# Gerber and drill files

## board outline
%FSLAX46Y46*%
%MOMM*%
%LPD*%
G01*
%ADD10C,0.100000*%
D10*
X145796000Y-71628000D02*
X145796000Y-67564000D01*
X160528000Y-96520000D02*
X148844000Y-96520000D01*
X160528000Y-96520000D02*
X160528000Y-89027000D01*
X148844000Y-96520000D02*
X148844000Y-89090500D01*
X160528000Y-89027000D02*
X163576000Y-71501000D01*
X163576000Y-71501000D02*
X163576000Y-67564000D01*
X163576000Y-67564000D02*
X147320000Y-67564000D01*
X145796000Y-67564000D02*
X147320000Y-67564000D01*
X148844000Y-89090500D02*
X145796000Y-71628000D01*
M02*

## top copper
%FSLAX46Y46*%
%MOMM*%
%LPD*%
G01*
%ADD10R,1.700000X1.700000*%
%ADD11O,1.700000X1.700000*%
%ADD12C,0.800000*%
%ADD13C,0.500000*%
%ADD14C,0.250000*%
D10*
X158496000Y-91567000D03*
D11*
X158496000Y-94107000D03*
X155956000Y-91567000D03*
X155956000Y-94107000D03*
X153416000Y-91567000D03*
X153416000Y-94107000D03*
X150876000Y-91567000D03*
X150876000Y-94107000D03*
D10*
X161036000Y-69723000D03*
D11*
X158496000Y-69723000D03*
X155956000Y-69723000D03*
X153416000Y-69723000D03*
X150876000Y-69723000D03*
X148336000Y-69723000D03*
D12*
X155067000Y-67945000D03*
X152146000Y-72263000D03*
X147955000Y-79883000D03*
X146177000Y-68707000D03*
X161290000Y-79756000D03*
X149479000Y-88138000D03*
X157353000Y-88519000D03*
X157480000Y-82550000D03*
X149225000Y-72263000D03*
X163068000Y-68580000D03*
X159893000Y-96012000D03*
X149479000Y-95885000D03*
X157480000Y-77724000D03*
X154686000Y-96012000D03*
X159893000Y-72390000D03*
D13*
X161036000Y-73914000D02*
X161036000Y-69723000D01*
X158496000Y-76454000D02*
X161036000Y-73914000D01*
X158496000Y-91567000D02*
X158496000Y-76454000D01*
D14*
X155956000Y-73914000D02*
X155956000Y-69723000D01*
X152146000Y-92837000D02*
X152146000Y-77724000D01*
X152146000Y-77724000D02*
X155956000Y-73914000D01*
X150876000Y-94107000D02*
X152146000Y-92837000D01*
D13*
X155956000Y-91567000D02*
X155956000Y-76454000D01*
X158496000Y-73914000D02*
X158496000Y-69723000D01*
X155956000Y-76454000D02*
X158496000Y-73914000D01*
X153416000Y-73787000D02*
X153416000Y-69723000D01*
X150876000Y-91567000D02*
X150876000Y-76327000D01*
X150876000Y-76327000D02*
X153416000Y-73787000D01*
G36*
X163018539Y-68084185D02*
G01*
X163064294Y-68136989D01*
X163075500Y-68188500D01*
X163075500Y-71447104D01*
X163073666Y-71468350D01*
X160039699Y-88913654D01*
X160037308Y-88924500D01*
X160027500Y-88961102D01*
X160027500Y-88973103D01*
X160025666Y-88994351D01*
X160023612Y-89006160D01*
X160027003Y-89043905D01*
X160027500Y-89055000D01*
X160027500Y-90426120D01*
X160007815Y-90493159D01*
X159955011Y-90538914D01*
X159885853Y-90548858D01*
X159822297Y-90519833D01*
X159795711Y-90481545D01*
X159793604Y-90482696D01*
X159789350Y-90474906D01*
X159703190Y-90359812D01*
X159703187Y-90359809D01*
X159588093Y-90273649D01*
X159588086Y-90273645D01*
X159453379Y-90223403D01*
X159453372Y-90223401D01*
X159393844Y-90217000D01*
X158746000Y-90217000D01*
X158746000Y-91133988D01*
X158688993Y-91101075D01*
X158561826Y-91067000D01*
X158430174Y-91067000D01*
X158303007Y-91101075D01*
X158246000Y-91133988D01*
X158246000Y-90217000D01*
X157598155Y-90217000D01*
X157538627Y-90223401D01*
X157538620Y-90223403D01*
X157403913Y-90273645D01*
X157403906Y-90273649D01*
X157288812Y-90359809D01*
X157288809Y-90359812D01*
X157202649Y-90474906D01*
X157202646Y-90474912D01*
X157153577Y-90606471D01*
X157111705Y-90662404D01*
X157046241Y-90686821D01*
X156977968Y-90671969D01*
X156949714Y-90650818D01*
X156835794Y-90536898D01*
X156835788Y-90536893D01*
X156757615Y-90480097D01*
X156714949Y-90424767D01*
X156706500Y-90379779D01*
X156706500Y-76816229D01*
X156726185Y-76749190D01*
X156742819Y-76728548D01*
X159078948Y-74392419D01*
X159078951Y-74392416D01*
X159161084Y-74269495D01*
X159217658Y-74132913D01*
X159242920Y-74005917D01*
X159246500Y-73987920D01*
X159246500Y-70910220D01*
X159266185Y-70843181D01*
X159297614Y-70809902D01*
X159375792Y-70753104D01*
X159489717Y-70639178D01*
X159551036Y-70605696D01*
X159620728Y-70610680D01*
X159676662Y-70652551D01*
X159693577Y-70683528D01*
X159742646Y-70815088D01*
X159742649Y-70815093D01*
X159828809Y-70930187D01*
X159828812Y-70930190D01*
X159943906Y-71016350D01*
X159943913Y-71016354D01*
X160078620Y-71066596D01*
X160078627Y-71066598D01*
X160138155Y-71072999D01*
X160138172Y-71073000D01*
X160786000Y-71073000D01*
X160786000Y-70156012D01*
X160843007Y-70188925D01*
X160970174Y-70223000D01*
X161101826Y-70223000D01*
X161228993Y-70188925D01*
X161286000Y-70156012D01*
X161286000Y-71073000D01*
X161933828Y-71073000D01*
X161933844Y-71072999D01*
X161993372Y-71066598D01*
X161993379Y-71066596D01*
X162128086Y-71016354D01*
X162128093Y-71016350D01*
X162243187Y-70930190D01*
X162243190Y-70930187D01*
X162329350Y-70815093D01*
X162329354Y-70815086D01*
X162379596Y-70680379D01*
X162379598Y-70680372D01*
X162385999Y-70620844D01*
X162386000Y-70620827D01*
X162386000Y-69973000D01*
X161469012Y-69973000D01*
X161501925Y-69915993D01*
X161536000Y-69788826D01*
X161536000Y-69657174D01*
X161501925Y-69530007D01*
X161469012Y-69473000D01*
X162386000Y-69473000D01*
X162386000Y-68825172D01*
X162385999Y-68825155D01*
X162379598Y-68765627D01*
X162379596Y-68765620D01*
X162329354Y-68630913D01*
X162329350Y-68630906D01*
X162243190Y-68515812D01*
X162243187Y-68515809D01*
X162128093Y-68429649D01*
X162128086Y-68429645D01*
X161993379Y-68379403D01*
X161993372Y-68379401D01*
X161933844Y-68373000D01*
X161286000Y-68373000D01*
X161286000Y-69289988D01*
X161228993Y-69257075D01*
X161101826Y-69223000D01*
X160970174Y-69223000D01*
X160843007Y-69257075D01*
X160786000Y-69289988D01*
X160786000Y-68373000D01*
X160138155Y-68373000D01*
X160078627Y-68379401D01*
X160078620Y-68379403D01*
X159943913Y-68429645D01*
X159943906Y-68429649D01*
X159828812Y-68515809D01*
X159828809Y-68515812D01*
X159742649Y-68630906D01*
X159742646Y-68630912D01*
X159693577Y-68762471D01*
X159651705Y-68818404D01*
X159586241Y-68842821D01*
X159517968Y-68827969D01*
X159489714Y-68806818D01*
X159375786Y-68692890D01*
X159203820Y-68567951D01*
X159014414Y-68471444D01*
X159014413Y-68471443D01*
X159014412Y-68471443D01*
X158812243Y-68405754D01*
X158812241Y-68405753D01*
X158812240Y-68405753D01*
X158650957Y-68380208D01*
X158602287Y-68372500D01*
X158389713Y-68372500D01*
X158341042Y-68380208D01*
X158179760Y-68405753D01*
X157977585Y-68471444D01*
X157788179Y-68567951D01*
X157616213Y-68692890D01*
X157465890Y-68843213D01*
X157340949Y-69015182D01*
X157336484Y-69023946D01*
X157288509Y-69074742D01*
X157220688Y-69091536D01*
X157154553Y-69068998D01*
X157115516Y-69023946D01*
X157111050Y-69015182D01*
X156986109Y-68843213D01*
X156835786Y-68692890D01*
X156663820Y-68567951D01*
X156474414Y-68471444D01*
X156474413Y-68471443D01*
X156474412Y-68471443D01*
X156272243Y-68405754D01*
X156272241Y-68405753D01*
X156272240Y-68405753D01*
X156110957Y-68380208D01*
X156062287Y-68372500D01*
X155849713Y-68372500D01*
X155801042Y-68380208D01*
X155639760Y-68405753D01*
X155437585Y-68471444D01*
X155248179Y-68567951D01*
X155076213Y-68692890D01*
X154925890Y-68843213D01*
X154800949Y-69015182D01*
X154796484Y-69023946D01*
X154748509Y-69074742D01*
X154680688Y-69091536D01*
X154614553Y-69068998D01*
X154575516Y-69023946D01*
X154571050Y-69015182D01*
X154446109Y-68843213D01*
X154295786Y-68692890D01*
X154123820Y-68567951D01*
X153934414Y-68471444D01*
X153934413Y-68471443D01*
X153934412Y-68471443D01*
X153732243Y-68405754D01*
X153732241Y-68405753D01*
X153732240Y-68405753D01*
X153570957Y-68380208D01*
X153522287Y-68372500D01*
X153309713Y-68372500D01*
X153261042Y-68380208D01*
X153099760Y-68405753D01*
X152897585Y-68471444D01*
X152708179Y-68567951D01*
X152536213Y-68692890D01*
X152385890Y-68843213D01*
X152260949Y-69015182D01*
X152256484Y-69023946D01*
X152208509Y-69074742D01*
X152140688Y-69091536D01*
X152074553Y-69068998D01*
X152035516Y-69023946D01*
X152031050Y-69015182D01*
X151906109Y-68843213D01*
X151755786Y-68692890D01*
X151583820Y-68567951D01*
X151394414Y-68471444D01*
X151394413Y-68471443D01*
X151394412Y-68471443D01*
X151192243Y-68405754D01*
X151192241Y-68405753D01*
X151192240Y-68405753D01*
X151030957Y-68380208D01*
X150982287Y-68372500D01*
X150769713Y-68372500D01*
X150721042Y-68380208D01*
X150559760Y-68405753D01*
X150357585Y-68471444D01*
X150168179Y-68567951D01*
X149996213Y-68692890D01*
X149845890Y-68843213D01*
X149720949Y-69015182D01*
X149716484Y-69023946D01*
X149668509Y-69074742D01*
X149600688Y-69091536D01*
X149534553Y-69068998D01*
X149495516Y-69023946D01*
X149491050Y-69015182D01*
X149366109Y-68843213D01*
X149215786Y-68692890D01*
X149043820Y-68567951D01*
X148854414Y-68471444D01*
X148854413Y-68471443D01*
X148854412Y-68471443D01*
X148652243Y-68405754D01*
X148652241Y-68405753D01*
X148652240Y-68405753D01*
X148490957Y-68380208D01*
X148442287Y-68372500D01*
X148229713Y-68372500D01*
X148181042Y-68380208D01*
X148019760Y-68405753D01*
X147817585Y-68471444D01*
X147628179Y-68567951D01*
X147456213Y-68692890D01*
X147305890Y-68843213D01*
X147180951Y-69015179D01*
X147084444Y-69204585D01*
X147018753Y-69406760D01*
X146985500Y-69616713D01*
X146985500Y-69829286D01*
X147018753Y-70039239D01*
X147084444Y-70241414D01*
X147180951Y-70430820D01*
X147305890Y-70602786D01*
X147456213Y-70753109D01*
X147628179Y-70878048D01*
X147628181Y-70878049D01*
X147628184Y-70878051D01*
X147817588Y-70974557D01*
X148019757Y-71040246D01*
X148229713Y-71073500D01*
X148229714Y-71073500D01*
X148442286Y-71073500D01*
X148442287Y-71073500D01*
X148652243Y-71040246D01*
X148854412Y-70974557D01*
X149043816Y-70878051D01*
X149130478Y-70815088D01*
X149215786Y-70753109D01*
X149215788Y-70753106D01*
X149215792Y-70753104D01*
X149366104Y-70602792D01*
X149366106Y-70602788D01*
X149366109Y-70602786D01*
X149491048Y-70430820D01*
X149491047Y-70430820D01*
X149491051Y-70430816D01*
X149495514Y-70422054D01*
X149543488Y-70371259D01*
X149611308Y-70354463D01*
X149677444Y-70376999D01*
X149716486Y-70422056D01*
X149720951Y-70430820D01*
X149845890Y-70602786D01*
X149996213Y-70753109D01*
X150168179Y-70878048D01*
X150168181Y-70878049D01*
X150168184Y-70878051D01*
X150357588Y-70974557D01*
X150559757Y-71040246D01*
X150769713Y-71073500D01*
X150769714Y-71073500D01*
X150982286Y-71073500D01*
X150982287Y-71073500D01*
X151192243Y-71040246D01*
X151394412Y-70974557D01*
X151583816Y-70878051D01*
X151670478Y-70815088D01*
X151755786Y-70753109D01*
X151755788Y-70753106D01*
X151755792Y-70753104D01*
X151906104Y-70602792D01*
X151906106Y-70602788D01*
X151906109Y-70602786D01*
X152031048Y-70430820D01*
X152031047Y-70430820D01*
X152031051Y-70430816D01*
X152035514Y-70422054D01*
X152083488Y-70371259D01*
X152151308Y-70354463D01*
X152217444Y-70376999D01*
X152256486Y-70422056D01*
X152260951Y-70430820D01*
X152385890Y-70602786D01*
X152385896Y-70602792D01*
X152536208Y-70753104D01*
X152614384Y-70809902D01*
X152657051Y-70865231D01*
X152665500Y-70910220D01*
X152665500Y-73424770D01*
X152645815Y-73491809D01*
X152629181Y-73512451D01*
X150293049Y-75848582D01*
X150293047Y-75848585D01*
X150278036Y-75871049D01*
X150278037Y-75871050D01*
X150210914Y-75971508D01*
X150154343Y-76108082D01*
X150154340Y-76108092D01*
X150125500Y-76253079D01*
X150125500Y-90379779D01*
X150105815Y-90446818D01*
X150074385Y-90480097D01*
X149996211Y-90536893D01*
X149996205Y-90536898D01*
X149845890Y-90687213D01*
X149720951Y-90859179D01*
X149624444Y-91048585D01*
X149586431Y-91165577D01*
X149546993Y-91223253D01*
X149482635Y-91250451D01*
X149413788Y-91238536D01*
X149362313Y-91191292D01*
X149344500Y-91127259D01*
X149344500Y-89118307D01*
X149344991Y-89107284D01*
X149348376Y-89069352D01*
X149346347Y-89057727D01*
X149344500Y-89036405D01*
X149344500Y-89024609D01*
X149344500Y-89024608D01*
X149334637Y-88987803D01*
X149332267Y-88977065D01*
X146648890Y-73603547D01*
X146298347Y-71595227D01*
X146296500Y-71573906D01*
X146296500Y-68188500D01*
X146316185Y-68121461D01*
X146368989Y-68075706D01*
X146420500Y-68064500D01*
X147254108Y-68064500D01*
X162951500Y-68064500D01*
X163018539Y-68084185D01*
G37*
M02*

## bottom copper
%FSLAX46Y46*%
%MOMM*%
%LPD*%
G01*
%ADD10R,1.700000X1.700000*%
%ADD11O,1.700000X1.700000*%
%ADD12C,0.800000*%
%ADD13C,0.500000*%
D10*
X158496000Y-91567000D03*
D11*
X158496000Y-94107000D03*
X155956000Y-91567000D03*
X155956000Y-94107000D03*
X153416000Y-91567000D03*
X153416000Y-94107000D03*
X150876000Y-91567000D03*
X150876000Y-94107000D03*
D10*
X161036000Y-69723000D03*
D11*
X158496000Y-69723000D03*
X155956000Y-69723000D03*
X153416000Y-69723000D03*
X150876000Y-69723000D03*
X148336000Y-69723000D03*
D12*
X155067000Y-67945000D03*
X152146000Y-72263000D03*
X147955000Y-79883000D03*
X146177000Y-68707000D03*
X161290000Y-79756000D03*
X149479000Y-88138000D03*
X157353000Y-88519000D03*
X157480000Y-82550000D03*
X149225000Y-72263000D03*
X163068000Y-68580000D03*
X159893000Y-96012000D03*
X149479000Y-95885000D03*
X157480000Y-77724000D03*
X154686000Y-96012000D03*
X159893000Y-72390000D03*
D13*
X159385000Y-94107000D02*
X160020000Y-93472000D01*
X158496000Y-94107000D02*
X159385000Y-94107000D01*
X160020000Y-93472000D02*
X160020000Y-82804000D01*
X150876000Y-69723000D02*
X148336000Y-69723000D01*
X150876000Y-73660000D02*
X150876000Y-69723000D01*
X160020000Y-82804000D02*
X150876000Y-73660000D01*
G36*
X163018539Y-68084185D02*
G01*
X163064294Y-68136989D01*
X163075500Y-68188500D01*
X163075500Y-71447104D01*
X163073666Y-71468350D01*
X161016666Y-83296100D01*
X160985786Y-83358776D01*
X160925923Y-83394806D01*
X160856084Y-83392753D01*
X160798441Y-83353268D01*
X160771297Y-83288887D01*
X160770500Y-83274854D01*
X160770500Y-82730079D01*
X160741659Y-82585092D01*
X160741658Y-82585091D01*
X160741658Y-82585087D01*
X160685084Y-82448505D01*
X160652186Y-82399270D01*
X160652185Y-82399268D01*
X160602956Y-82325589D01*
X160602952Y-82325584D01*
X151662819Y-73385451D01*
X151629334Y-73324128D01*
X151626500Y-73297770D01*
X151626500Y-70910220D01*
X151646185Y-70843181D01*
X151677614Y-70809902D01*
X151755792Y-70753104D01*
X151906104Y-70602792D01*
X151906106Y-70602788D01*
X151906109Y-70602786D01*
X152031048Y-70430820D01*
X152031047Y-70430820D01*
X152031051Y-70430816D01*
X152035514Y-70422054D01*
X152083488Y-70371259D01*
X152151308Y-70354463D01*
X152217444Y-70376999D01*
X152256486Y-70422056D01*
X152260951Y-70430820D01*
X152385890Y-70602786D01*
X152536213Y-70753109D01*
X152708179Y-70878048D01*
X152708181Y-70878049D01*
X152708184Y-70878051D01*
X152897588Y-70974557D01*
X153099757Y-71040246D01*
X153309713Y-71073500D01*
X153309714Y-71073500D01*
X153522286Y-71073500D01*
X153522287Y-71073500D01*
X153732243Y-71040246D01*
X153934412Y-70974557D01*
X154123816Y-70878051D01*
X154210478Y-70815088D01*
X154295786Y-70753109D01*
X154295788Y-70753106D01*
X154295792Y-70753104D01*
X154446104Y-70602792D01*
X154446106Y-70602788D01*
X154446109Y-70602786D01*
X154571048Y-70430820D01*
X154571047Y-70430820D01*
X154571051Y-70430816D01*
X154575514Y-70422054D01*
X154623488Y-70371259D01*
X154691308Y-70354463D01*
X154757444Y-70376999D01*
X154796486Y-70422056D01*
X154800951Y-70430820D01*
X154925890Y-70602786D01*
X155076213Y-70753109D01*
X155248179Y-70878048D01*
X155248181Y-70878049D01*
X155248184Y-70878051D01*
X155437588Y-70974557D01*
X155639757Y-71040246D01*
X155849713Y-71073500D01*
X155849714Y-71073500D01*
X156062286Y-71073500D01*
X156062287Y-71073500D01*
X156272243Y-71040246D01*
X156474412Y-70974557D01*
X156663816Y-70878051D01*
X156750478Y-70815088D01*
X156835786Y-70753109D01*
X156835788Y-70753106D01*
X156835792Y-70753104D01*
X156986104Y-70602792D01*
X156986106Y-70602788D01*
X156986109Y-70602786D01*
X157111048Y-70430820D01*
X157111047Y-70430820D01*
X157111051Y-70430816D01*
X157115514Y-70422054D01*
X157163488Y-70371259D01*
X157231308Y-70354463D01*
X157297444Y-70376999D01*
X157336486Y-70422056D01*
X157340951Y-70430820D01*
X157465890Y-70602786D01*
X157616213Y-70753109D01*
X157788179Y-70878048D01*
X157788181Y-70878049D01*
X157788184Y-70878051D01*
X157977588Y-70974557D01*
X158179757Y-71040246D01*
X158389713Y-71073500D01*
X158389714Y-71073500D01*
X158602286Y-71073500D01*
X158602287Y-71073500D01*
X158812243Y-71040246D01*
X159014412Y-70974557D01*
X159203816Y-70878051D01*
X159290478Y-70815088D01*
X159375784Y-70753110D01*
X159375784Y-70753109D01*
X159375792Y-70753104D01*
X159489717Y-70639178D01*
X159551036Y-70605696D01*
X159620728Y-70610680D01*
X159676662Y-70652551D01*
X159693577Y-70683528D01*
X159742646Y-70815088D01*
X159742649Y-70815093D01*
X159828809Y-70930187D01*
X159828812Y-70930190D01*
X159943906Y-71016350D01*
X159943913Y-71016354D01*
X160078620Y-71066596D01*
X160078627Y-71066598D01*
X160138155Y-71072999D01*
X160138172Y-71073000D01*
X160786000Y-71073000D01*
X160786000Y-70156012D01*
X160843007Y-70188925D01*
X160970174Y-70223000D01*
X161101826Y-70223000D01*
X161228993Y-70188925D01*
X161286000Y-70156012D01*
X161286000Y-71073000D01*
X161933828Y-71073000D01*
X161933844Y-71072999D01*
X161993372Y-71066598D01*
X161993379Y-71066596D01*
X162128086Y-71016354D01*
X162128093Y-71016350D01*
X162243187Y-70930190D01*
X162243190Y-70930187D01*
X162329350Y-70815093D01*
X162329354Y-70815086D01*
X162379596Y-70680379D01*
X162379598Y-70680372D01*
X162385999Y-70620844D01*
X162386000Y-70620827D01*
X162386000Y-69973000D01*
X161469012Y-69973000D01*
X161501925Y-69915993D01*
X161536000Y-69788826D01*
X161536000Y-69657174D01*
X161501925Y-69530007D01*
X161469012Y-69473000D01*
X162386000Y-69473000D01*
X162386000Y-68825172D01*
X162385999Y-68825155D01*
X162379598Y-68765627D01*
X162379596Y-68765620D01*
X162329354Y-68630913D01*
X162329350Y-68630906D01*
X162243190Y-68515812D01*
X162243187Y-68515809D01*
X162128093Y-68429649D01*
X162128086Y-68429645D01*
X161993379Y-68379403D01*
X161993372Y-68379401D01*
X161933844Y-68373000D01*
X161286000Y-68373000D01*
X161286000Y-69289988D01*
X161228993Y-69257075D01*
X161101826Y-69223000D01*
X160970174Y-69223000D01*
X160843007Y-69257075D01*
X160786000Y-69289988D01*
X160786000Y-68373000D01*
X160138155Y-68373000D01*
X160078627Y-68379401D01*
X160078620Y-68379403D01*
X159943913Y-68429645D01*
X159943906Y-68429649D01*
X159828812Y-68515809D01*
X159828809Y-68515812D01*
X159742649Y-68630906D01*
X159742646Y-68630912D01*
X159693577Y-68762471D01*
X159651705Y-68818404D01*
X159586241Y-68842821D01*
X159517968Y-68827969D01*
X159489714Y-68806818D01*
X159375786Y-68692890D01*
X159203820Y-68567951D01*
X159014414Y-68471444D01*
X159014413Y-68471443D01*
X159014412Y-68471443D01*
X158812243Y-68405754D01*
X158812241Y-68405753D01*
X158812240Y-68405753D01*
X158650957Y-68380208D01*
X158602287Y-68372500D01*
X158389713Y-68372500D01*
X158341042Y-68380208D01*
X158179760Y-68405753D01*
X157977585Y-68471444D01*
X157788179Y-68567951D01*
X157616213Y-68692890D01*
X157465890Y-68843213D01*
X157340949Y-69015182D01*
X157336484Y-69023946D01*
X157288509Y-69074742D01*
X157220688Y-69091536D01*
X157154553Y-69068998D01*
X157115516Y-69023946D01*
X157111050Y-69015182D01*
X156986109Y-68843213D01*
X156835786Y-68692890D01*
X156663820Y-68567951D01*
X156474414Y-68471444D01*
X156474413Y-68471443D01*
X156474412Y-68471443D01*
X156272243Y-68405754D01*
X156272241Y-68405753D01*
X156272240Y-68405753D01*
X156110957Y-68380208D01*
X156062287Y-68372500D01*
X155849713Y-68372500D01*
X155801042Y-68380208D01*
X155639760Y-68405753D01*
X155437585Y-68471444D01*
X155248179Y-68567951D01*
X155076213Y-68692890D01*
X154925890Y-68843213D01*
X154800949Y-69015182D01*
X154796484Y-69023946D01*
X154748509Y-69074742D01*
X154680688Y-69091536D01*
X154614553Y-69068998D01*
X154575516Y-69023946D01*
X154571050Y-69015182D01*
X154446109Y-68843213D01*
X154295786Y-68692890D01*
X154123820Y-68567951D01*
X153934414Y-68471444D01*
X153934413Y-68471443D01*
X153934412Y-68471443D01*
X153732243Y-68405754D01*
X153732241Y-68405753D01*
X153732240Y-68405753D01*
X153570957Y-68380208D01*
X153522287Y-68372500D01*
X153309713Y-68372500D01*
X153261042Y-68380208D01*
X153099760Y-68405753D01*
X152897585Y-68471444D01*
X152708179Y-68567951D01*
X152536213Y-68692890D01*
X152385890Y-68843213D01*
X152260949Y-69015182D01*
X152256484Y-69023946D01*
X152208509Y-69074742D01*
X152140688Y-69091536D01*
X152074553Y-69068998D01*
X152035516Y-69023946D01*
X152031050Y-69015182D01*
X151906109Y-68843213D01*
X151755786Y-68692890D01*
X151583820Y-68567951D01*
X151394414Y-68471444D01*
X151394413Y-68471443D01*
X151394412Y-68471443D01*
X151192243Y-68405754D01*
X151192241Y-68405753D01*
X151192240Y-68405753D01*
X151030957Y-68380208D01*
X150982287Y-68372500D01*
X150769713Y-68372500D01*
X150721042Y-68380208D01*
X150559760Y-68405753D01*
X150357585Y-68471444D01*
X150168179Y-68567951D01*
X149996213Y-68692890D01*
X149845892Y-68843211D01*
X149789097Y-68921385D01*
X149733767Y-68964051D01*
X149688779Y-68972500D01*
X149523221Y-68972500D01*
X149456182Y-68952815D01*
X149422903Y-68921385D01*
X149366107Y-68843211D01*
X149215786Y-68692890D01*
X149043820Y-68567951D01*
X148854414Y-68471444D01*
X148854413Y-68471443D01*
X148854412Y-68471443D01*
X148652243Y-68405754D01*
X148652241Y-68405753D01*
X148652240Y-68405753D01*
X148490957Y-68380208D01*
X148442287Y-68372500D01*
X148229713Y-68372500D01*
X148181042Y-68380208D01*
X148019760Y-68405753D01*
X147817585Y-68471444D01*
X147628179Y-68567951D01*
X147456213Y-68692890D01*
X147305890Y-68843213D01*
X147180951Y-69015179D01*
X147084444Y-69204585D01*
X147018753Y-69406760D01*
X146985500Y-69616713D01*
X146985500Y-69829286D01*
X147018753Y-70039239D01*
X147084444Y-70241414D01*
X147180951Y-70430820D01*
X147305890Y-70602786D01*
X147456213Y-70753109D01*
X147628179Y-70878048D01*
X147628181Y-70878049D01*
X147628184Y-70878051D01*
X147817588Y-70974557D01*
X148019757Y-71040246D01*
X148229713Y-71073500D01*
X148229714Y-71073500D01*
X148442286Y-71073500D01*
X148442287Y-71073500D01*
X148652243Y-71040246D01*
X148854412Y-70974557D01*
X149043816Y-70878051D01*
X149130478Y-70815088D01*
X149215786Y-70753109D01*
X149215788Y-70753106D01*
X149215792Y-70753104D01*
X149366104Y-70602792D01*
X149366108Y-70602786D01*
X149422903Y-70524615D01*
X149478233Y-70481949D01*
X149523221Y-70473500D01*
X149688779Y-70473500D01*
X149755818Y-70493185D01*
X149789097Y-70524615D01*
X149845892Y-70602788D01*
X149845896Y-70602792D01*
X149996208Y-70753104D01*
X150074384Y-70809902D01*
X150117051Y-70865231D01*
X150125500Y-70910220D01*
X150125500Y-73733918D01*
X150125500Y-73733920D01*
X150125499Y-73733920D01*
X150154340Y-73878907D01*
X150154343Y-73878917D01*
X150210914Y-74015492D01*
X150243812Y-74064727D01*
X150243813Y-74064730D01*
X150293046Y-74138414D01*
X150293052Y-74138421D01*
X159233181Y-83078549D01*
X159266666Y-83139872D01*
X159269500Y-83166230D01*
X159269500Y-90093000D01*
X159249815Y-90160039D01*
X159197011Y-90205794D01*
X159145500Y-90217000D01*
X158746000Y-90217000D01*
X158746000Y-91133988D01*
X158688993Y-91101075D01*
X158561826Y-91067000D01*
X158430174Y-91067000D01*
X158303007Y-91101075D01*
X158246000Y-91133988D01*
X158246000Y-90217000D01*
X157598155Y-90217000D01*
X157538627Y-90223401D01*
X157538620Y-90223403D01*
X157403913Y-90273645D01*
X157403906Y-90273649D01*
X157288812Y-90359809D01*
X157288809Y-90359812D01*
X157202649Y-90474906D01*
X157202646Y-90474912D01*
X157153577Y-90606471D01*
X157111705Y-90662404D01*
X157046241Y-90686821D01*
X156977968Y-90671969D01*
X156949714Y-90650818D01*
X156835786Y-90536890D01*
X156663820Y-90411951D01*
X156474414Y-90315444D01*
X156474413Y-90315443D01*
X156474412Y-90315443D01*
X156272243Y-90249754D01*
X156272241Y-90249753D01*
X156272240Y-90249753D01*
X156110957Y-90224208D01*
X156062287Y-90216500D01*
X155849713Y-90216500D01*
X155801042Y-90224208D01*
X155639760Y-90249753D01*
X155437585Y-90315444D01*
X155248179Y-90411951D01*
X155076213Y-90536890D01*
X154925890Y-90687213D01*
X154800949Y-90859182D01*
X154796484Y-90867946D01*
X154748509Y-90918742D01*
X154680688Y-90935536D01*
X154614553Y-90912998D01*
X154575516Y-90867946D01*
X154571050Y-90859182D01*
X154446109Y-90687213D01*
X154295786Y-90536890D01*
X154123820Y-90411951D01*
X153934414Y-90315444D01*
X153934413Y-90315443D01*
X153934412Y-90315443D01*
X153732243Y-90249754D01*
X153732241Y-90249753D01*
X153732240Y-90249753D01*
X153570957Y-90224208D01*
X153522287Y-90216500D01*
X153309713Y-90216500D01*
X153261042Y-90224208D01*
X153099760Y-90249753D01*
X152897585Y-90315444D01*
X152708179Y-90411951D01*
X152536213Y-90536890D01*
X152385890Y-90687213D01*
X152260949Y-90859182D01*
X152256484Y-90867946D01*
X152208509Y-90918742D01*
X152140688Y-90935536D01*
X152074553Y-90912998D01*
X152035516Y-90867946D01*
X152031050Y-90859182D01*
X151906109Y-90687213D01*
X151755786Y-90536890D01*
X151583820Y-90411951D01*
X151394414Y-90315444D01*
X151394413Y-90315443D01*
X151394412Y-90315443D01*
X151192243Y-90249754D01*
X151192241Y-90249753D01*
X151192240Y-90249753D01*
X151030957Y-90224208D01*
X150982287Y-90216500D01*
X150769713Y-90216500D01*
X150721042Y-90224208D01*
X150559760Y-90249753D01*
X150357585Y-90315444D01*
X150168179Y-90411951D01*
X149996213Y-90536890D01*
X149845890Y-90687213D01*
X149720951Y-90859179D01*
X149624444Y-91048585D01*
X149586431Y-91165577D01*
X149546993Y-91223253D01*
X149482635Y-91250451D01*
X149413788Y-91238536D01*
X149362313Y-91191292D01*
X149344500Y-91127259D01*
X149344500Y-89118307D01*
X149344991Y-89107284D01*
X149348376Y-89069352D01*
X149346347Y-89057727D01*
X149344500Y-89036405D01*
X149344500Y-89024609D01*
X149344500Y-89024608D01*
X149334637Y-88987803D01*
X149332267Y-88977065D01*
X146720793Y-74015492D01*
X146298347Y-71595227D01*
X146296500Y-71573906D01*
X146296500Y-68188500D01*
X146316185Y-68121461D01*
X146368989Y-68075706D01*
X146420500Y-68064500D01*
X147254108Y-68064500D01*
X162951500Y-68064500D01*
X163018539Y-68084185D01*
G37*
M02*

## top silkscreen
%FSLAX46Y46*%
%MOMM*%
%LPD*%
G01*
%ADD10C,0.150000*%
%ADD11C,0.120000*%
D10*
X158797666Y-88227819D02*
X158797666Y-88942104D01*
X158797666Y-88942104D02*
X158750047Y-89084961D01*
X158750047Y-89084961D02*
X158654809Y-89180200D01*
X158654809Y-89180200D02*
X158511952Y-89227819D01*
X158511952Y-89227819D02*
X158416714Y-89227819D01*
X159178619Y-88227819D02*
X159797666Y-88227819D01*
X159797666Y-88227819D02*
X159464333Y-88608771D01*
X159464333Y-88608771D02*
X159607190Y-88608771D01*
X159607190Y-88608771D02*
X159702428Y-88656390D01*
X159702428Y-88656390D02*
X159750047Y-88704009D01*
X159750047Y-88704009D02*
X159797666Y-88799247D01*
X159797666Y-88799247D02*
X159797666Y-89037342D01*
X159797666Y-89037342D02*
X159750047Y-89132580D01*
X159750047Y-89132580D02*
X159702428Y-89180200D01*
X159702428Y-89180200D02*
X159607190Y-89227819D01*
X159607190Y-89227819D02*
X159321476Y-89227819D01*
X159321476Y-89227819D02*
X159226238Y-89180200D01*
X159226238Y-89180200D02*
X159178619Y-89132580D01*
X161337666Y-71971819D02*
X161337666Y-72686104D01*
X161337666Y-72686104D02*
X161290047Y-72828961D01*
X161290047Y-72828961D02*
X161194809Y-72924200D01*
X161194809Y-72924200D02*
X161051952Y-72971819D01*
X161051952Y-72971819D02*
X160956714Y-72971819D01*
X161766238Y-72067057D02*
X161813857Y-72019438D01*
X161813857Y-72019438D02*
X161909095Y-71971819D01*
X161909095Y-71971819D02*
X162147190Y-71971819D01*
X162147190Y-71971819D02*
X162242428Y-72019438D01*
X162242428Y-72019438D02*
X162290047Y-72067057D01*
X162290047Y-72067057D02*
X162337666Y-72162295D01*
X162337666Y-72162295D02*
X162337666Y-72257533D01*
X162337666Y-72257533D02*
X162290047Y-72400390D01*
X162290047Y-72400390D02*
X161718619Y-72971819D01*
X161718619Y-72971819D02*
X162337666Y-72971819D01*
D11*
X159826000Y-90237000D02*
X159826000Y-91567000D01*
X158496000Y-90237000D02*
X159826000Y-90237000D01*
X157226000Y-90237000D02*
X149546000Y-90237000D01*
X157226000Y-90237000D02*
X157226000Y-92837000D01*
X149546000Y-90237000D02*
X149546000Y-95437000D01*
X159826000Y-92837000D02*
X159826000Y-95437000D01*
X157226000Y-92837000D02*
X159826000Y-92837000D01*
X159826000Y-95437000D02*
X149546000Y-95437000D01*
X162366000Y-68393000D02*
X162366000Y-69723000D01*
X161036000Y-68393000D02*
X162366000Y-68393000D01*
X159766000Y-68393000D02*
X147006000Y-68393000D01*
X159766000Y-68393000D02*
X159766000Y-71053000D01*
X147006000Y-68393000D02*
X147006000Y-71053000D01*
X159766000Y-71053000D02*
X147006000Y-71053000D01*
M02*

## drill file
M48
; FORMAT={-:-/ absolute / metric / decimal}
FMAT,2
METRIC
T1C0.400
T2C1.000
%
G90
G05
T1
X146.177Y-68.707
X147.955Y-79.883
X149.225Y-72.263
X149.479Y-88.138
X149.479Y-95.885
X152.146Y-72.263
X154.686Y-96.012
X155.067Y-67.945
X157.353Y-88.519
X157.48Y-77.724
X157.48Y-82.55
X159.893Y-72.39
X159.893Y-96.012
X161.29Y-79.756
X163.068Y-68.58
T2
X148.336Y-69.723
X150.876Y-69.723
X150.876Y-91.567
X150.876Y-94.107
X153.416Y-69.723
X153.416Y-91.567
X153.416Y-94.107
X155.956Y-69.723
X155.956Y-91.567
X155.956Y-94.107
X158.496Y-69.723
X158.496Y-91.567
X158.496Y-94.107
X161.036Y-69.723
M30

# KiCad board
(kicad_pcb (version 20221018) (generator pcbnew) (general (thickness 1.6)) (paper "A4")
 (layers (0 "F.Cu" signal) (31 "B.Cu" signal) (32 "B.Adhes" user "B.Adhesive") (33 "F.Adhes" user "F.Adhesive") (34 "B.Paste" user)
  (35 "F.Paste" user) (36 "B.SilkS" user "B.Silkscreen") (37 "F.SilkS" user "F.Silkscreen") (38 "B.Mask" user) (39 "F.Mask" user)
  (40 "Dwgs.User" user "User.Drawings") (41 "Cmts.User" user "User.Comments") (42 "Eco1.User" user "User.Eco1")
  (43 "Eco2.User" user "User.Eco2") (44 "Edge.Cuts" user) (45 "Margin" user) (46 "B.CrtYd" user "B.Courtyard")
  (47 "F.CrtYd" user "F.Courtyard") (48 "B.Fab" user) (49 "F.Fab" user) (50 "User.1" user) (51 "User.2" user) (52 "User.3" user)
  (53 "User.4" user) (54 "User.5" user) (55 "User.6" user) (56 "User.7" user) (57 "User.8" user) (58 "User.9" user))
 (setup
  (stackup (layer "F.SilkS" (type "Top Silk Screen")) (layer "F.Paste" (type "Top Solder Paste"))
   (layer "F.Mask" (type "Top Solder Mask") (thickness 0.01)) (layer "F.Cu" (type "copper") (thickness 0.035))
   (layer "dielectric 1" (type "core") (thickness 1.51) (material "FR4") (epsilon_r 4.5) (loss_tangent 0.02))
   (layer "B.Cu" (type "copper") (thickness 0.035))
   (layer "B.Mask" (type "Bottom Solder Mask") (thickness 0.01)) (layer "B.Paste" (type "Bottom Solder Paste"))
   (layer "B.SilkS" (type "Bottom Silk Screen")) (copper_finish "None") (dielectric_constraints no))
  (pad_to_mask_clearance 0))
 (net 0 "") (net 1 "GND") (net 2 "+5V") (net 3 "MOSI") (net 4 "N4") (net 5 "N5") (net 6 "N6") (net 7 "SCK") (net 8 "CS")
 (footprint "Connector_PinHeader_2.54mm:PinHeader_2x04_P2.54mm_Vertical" (layer "F.Cu") (at 158.496 91.567 -90)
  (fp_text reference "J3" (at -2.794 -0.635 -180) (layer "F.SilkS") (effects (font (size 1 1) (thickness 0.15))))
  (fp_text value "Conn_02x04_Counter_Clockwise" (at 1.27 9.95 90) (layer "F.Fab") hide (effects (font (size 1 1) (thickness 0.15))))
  (fp_line (start -1.33 -1.33) (end 0 -1.33) (stroke (width 0.12) (type solid)) (layer "F.SilkS"))
  (fp_line (start -1.33 0) (end -1.33 -1.33) (stroke (width 0.12) (type solid)) (layer "F.SilkS"))
  (fp_line (start -1.33 1.27) (end -1.33 8.95) (stroke (width 0.12) (type solid)) (layer "F.SilkS"))
  (fp_line (start -1.33 1.27) (end 1.27 1.27) (stroke (width 0.12) (type solid)) (layer "F.SilkS"))
  (fp_line (start -1.33 8.95) (end 3.87 8.95) (stroke (width 0.12) (type solid)) (layer "F.SilkS"))
  (fp_line (start 1.27 -1.33) (end 3.87 -1.33) (stroke (width 0.12) (type solid)) (layer "F.SilkS"))
  (fp_line (start 1.27 1.27) (end 1.27 -1.33) (stroke (width 0.12) (type solid)) (layer "F.SilkS"))
  (fp_line (start 3.87 -1.33) (end 3.87 8.95) (stroke (width 0.12) (type solid)) (layer "F.SilkS"))
  (pad "1" thru_hole rect (at 0 0 270) (size 1.7 1.7) (drill 1) (layers "*.Cu" "*.Mask") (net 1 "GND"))
  (pad "2" thru_hole oval (at 2.54 0 270) (size 1.7 1.7) (drill 1) (layers "*.Cu" "*.Mask") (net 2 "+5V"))
  (pad "3" thru_hole oval (at 0 2.54 270) (size 1.7 1.7) (drill 1) (layers "*.Cu" "*.Mask") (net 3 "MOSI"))
  (pad "4" thru_hole oval (at 2.54 2.54 270) (size 1.7 1.7) (drill 1) (layers "*.Cu" "*.Mask") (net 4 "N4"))
  (pad "5" thru_hole oval (at 0 5.08 270) (size 1.7 1.7) (drill 1) (layers "*.Cu" "*.Mask") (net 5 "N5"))
  (pad "6" thru_hole oval (at 2.54 5.08 270) (size 1.7 1.7) (drill 1) (layers "*.Cu" "*.Mask") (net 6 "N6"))
  (pad "7" thru_hole oval (at 0 7.62 270) (size 1.7 1.7) (drill 1) (layers "*.Cu" "*.Mask") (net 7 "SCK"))
  (pad "8" thru_hole oval (at 2.54 7.62 270) (size 1.7 1.7) (drill 1) (layers "*.Cu" "*.Mask") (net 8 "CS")))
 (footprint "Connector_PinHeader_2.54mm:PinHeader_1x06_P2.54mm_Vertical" (layer "F.Cu") (at 161.036 69.723 -90)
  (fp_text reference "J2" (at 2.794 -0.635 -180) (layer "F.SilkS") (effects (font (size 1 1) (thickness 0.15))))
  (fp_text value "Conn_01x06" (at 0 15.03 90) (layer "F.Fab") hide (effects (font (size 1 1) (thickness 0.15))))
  (fp_line (start -1.33 -1.33) (end 0 -1.33) (stroke (width 0.12) (type solid)) (layer "F.SilkS"))
  (fp_line (start -1.33 0) (end -1.33 -1.33) (stroke (width 0.12) (type solid)) (layer "F.SilkS"))
  (fp_line (start -1.33 1.27) (end -1.33 14.03) (stroke (width 0.12) (type solid)) (layer "F.SilkS"))
  (fp_line (start -1.33 1.27) (end 1.33 1.27) (stroke (width 0.12) (type solid)) (layer "F.SilkS"))
  (fp_line (start -1.33 14.03) (end 1.33 14.03) (stroke (width 0.12) (type solid)) (layer "F.SilkS"))
  (fp_line (start 1.33 1.27) (end 1.33 14.03) (stroke (width 0.12) (type solid)) (layer "F.SilkS"))
  (pad "1" thru_hole rect (at 0 0 270) (size 1.7 1.7) (drill 1) (layers "*.Cu" "*.Mask") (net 1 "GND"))
  (pad "2" thru_hole oval (at 0 2.54 270) (size 1.7 1.7) (drill 1) (layers "*.Cu" "*.Mask") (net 3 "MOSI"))
  (pad "3" thru_hole oval (at 0 5.08 270) (size 1.7 1.7) (drill 1) (layers "*.Cu" "*.Mask") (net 8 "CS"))
  (pad "4" thru_hole oval (at 0 7.62 270) (size 1.7 1.7) (drill 1) (layers "*.Cu" "*.Mask") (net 7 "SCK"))
  (pad "5" thru_hole oval (at 0 10.16 270) (size 1.7 1.7) (drill 1) (layers "*.Cu" "*.Mask") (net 2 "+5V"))
  (pad "6" thru_hole oval (at 0 12.7 270) (size 1.7 1.7) (drill 1) (layers "*.Cu" "*.Mask") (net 2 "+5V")))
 (gr_line (start 145.796 71.628) (end 145.796 67.564) (stroke (width 0.1) (type default)) (layer "Edge.Cuts"))
 (gr_line (start 160.528 96.52) (end 148.844 96.52) (stroke (width 0.1) (type default)) (layer "Edge.Cuts"))
 (gr_line (start 160.528 96.52) (end 160.528 89.027) (stroke (width 0.1) (type default)) (layer "Edge.Cuts"))
 (gr_line (start 148.844 96.52) (end 148.844 89.0905) (stroke (width 0.1) (type default)) (layer "Edge.Cuts"))
 (gr_line (start 160.528 89.027) (end 163.576 71.501) (stroke (width 0.1) (type default)) (layer "Edge.Cuts"))
 (gr_line (start 163.576 71.501) (end 163.576 67.564) (stroke (width 0.1) (type default)) (layer "Edge.Cuts"))
 (gr_line (start 163.576 67.564) (end 147.32 67.564) (stroke (width 0.1) (type default)) (layer "Edge.Cuts"))
 (gr_line (start 145.796 67.564) (end 147.32 67.564) (stroke (width 0.1) (type default)) (layer "Edge.Cuts"))
 (gr_line (start 148.844 89.0905) (end 145.796 71.628) (stroke (width 0.1) (type default)) (layer "Edge.Cuts"))
 (segment (start 161.036 73.914) (end 161.036 69.723) (width 0.5) (layer "F.Cu") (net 1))
 (segment (start 158.496 76.454) (end 161.036 73.914) (width 0.5) (layer "F.Cu") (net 1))
 (segment (start 158.496 91.567) (end 158.496 76.454) (width 0.5) (layer "F.Cu") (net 1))
 (via (at 155.067 67.945) (size 0.8) (drill 0.4) (layers "F.Cu" "B.Cu") (free) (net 1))
 (via (at 152.146 72.263) (size 0.8) (drill 0.4) (layers "F.Cu" "B.Cu") (free) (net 1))
 (via (at 147.955 79.883) (size 0.8) (drill 0.4) (layers "F.Cu" "B.Cu") (free) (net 1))
 (via (at 146.177 68.707) (size 0.8) (drill 0.4) (layers "F.Cu" "B.Cu") (free) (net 1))
 (via (at 161.29 79.756) (size 0.8) (drill 0.4) (layers "F.Cu" "B.Cu") (free) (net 1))
 (via (at 149.479 88.138) (size 0.8) (drill 0.4) (layers "F.Cu" "B.Cu") (free) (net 1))
 (via (at 157.353 88.519) (size 0.8) (drill 0.4) (layers "F.Cu" "B.Cu") (free) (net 1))
 (via (at 157.48 82.55) (size 0.8) (drill 0.4) (layers "F.Cu" "B.Cu") (free) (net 1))
 (via (at 149.225 72.263) (size 0.8) (drill 0.4) (layers "F.Cu" "B.Cu") (free) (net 1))
 (via (at 163.068 68.58) (size 0.8) (drill 0.4) (layers "F.Cu" "B.Cu") (free) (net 1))
 (via (at 159.893 96.012) (size 0.8) (drill 0.4) (layers "F.Cu" "B.Cu") (free) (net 1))
 (via (at 149.479 95.885) (size 0.8) (drill 0.4) (layers "F.Cu" "B.Cu") (free) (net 1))
 (via (at 157.48 77.724) (size 0.8) (drill 0.4) (layers "F.Cu" "B.Cu") (free) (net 1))
 (via (at 154.686 96.012) (size 0.8) (drill 0.4) (layers "F.Cu" "B.Cu") (free) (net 1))
 (via (at 159.893 72.39) (size 0.8) (drill 0.4) (layers "F.Cu" "B.Cu") (free) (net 1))
 (segment (start 155.956 73.914) (end 155.956 69.723) (width 0.25) (layer "F.Cu") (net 8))
 (segment (start 152.146 92.837) (end 152.146 77.724) (width 0.25) (layer "F.Cu") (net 8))
 (segment (start 152.146 77.724) (end 155.956 73.914) (width 0.25) (layer "F.Cu") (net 8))
 (segment (start 150.876 94.107) (end 152.146 92.837) (width 0.25) (layer "F.Cu") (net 8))
 (segment (start 155.956 91.567) (end 155.956 76.454) (width 0.5) (layer "F.Cu") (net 3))
 (segment (start 158.496 73.914) (end 158.496 69.723) (width 0.5) (layer "F.Cu") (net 3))
 (segment (start 155.956 76.454) (end 158.496 73.914) (width 0.5) (layer "F.Cu") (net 3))
 (segment (start 153.416 73.787) (end 153.416 69.723) (width 0.5) (layer "F.Cu") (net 7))
 (segment (start 150.876 91.567) (end 150.876 76.327) (width 0.5) (layer "F.Cu") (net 7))
 (segment (start 150.876 76.327) (end 153.416 73.787) (width 0.5) (layer "F.Cu") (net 7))
 (segment (start 159.385 94.107) (end 160.02 93.472) (width 0.5) (layer "B.Cu") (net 2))
 (segment (start 158.496 94.107) (end 159.385 94.107) (width 0.5) (layer "B.Cu") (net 2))
 (segment (start 160.02 93.472) (end 160.02 82.804) (width 0.5) (layer "B.Cu") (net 2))
 (segment (start 150.876 69.723) (end 148.336 69.723) (width 0.5) (layer "B.Cu") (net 2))
 (segment (start 150.876 73.66) (end 150.876 69.723) (width 0.5) (layer "B.Cu") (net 2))
 (segment (start 160.02 82.804) (end 150.876 73.66) (width 0.5) (layer "B.Cu") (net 2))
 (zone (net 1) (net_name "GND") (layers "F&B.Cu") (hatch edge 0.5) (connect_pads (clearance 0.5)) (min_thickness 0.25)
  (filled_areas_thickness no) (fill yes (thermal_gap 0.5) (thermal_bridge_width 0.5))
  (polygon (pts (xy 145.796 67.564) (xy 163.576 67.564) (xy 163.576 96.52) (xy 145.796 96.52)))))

